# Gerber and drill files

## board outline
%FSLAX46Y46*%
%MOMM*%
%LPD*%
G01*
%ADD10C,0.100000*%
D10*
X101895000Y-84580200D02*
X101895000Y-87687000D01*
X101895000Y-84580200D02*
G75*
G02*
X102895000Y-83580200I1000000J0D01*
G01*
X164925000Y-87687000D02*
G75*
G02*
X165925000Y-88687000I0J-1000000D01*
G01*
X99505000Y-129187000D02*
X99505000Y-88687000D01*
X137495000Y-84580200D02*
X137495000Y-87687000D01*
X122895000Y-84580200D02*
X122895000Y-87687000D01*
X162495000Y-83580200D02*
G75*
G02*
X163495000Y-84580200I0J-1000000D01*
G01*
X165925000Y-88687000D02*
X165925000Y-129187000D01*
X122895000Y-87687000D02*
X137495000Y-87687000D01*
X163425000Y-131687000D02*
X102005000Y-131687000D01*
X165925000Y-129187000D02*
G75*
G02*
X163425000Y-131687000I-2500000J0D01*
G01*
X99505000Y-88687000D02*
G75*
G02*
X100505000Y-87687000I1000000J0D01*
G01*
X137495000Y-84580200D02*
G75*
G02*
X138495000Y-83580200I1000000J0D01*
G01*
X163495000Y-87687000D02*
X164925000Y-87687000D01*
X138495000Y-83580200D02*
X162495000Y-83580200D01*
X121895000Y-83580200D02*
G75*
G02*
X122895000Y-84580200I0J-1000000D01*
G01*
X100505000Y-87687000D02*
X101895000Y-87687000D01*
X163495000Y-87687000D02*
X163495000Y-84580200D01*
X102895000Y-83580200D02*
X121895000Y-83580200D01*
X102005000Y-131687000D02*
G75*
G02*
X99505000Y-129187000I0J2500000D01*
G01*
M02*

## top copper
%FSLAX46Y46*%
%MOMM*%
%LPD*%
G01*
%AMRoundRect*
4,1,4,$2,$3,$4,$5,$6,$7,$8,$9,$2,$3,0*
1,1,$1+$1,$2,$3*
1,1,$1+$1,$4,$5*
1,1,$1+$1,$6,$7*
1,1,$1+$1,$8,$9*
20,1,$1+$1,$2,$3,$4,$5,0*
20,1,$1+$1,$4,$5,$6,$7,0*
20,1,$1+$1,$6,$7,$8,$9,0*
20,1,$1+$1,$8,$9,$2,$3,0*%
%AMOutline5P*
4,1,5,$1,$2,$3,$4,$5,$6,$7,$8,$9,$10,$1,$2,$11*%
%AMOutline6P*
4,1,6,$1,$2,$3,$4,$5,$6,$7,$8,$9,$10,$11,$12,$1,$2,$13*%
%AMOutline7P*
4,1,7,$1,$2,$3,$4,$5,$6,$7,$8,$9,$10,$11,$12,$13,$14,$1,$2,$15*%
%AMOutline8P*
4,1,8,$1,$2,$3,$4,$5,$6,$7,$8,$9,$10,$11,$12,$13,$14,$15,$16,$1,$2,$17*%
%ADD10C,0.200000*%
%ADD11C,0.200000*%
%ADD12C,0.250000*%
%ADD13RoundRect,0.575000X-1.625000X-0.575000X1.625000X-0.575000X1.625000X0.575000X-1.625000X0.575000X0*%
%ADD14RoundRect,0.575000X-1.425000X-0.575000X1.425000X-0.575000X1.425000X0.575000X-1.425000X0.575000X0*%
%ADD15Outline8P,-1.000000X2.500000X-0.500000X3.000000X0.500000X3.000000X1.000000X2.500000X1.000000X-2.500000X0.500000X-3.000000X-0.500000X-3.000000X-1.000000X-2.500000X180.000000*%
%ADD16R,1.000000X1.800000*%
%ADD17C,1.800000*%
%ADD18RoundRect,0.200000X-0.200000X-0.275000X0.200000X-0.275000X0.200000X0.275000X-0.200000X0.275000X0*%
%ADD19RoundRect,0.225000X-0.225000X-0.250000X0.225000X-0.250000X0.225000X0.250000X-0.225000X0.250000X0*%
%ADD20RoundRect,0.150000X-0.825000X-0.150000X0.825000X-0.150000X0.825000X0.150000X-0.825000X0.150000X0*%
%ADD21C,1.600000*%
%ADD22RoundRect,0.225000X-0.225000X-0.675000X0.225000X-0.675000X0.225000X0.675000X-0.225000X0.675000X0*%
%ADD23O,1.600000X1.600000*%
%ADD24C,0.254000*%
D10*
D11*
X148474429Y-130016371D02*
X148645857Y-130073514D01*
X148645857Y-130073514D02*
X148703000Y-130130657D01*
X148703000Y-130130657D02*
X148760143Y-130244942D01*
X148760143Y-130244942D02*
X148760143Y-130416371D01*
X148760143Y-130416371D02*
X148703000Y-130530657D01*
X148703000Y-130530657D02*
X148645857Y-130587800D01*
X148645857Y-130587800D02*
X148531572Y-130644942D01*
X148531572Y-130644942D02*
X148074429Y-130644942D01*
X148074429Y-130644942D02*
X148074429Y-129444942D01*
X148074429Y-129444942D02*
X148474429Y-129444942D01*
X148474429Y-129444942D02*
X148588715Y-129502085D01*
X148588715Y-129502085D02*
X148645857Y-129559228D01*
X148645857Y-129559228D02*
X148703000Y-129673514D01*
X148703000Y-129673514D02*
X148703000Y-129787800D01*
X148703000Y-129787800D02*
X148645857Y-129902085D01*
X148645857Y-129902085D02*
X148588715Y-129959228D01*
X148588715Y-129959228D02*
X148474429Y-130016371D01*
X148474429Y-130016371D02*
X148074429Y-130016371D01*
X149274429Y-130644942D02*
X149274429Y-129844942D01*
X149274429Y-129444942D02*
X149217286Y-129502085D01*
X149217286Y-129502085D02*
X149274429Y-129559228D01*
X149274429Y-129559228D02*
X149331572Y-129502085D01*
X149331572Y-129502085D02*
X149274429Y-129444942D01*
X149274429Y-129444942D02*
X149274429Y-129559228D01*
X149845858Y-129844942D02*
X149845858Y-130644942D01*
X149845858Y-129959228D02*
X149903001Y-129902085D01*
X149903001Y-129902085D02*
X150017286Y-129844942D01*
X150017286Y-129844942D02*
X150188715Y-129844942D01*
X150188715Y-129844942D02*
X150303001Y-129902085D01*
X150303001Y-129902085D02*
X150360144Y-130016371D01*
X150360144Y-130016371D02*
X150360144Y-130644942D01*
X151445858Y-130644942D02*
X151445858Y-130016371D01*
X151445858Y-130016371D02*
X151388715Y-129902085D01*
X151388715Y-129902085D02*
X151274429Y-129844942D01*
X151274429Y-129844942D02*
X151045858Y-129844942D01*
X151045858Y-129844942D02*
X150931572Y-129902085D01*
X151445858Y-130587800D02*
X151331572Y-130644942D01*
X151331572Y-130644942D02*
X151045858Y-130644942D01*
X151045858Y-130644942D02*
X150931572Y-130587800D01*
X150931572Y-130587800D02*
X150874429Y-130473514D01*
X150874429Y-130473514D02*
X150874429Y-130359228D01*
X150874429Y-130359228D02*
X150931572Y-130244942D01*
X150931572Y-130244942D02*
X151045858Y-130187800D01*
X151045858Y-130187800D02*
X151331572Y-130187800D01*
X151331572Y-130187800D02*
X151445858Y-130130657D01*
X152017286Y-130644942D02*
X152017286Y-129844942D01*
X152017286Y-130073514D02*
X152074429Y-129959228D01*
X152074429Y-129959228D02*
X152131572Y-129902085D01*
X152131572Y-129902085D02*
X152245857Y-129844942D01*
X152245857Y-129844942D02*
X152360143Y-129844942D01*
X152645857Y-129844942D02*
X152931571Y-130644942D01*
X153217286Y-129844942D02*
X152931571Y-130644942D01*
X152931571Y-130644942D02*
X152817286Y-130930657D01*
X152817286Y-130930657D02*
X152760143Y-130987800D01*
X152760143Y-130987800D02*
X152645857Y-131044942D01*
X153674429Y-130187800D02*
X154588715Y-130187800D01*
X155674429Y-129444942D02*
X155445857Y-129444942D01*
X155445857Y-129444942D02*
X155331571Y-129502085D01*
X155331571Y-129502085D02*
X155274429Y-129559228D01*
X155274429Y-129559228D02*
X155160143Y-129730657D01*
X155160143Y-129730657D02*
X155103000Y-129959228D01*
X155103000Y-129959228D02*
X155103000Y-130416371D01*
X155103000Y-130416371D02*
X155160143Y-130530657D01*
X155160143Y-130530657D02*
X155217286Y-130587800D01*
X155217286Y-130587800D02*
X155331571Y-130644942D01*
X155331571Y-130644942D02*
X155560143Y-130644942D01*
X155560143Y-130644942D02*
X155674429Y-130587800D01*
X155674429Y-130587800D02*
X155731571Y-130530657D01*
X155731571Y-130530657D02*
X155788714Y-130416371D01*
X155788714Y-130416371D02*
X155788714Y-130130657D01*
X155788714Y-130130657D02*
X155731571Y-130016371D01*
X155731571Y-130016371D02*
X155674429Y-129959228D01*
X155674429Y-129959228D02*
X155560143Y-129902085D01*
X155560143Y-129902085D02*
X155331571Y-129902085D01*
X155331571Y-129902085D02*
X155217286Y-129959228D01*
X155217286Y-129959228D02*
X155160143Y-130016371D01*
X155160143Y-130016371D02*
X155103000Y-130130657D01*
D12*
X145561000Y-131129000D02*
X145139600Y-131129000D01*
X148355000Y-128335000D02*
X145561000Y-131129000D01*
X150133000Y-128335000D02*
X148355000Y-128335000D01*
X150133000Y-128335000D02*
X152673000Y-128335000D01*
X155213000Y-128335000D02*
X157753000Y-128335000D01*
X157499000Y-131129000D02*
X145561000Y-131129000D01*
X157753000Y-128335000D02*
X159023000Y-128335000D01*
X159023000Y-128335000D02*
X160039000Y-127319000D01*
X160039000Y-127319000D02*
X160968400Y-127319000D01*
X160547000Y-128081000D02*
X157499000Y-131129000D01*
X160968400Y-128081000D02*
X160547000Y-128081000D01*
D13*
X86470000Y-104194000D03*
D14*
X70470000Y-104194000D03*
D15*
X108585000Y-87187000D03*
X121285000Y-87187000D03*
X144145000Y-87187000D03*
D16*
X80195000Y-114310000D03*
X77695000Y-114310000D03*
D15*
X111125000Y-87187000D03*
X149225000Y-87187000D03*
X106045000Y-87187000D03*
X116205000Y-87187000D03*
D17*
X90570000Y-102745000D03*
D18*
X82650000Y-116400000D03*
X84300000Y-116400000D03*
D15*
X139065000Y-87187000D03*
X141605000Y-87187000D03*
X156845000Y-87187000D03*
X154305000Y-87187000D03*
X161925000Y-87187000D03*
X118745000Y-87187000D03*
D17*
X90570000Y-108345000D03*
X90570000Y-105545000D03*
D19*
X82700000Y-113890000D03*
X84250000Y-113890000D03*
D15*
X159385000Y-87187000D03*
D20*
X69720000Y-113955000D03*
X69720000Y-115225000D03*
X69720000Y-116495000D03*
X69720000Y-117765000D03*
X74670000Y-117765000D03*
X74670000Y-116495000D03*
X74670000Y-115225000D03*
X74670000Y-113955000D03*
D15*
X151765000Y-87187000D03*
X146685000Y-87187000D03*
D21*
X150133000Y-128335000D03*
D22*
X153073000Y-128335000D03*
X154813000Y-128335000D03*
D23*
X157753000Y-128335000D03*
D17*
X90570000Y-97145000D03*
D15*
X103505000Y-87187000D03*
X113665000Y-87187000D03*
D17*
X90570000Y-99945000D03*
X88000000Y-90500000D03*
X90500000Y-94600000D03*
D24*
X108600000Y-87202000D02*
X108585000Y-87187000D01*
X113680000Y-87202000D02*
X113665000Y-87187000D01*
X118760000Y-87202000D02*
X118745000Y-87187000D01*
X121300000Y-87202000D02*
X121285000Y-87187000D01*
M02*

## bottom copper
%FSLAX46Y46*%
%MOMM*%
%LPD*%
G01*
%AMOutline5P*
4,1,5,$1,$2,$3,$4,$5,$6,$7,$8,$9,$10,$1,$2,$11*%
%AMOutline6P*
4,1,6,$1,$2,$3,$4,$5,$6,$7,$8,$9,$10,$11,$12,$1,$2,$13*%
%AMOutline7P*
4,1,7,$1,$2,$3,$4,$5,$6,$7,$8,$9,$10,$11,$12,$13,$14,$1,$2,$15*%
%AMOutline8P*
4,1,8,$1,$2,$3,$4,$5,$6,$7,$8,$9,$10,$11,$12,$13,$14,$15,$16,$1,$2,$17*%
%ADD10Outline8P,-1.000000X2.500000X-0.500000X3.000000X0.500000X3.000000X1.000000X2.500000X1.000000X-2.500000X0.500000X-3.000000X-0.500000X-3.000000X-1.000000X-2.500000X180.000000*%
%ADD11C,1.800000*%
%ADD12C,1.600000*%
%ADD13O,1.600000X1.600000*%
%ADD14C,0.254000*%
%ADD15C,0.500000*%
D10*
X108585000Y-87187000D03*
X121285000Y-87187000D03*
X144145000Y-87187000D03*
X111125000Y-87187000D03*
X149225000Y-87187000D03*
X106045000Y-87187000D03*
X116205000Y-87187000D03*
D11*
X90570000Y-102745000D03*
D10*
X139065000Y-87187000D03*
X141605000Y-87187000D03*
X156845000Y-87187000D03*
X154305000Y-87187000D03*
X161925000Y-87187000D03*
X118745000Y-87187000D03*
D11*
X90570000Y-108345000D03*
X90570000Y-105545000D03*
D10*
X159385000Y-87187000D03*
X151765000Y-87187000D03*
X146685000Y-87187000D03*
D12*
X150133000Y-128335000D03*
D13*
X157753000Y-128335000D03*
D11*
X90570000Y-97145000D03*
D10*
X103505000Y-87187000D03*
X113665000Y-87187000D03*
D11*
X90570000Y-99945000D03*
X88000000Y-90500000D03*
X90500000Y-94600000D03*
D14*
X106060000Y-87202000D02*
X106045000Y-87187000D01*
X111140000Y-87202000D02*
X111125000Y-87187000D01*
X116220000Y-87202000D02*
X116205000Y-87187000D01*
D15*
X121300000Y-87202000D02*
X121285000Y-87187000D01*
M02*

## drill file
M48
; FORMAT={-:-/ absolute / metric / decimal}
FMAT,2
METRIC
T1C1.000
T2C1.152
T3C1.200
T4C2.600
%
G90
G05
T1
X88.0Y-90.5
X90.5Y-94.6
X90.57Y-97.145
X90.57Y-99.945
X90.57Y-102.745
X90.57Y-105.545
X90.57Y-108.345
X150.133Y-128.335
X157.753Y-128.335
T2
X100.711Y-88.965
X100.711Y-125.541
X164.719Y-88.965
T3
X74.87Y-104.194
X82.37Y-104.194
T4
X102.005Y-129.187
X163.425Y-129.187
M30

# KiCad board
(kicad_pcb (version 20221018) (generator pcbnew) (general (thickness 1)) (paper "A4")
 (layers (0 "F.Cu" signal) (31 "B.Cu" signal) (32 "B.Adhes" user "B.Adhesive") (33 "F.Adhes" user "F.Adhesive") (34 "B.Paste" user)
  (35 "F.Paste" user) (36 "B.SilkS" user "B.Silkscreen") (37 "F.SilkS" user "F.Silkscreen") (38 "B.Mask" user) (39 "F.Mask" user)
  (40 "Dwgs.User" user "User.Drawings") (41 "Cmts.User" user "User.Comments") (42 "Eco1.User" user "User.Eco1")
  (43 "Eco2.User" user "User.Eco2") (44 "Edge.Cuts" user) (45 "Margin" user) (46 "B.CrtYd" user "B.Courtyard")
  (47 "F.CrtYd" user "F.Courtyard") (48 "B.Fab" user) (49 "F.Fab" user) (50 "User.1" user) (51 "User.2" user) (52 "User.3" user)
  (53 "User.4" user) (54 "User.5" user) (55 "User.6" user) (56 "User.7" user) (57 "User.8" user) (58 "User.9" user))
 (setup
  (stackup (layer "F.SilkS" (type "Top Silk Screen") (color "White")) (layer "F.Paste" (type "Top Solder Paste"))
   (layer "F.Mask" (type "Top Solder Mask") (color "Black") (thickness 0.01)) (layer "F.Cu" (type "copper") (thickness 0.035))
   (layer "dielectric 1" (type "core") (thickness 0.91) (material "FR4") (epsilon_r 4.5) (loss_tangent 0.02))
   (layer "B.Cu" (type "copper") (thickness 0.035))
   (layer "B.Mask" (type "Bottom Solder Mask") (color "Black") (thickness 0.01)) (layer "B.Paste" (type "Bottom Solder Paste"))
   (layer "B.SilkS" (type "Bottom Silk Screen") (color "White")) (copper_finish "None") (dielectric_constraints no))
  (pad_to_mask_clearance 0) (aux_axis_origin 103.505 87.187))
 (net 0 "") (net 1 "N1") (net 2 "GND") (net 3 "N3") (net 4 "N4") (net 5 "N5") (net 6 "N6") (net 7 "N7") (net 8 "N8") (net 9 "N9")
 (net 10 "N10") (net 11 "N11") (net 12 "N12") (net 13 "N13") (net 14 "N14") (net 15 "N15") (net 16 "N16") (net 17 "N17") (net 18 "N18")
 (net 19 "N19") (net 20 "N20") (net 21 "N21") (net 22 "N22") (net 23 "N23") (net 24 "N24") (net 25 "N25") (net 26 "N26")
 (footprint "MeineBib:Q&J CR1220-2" (layer "F.Cu") (at 78.47 104.194)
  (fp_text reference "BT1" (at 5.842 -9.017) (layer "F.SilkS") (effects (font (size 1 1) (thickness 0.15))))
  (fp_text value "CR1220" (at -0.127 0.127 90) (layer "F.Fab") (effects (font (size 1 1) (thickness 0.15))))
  (pad "" np_thru_hole circle (at -3.6 0) (size 1.2 1.2) (drill 1.2) (layers "F&B.Cu" "*.Mask"))
  (pad "" np_thru_hole circle (at 3.9 0) (size 1.2 1.2) (drill 1.2) (layers "F&B.Cu" "*.Mask"))
  (pad "1" smd roundrect (at 8 0) (size 4.4 2.3) (layers "F.Cu" "F.Paste" "F.Mask") (roundrect_rratio 0.25) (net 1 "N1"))
  (pad "2" smd roundrect (at -8 0) (size 4 2.3) (layers "F.Cu" "F.Paste" "F.Mask") (roundrect_rratio 0.25) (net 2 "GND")))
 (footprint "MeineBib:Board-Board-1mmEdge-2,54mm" (layer "F.Cu") (at 108.585 87.187)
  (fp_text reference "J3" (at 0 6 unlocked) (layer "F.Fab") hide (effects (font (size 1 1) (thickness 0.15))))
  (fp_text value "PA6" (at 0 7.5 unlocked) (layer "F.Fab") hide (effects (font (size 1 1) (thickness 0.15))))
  (pad "1" smd roundrect (at 0 0 180) (size 2 6) (layers "F.Cu" "F.Paste" "F.Mask") (roundrect_rratio 0) (chamfer_ratio 0.25)
   (chamfer top_left top_right bottom_left bottom_right) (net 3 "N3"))
  (pad "1" smd roundrect (at 0 0 180) (size 2 6) (layers "B.Cu" "B.Paste" "B.Mask") (roundrect_rratio 0) (chamfer_ratio 0.25)
   (chamfer top_left top_right bottom_left bottom_right) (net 3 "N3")))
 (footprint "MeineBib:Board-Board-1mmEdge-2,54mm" (layer "F.Cu") (at 121.285 87.187)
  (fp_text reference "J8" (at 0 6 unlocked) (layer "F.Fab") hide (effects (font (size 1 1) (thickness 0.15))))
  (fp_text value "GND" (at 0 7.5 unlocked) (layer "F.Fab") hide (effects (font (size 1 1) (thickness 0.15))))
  (pad "1" smd roundrect (at 0 0 180) (size 2 6) (layers "F.Cu" "F.Paste" "F.Mask") (roundrect_rratio 0) (chamfer_ratio 0.25)
   (chamfer top_left top_right bottom_left bottom_right) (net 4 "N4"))
  (pad "1" smd roundrect (at 0 0 180) (size 2 6) (layers "B.Cu" "B.Paste" "B.Mask") (roundrect_rratio 0) (chamfer_ratio 0.25)
   (chamfer top_left top_right bottom_left bottom_right) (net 4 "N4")))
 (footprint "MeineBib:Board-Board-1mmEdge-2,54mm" (layer "F.Cu") (at 144.145 87.187)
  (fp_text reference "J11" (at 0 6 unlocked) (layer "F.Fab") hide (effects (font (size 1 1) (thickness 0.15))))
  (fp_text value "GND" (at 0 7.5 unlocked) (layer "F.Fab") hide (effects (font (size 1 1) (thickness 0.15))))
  (pad "1" smd roundrect (at 0 0 180) (size 2 6) (layers "F.Cu" "F.Paste" "F.Mask") (roundrect_rratio 0) (chamfer_ratio 0.25)
   (chamfer top_left top_right bottom_left bottom_right) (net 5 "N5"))
  (pad "1" smd roundrect (at 0 0 180) (size 2 6) (layers "B.Cu" "B.Paste" "B.Mask") (roundrect_rratio 0) (chamfer_ratio 0.25)
   (chamfer top_left top_right bottom_left bottom_right) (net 5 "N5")))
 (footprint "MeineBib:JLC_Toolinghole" (layer "F.Cu") (at 164.719 88.965)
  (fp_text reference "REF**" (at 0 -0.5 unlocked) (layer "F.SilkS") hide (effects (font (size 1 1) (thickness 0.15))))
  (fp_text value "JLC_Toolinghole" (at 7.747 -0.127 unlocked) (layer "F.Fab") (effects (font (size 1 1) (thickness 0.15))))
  (pad "" np_thru_hole circle (at 0 0) (size 1.3 1.3) (drill 1.152) (layers "*.Mask")))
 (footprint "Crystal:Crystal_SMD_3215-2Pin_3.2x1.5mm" (layer "F.Cu") (at 78.945 114.31)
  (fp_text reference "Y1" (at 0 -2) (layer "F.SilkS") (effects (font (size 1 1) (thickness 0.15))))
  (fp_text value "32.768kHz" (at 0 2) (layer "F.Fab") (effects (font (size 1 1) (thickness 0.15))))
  (pad "1" smd rect (at 1.25 0) (size 1 1.8) (layers "F.Cu" "F.Paste" "F.Mask") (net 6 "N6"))
  (pad "2" smd rect (at -1.25 0) (size 1 1.8) (layers "F.Cu" "F.Paste" "F.Mask") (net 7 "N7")))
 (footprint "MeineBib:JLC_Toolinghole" (layer "F.Cu") (at 100.711 125.541)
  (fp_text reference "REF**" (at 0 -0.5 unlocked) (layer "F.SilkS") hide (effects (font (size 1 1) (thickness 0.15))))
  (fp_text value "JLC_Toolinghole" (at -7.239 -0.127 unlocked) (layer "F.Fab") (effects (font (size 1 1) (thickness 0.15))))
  (pad "" np_thru_hole circle (at 0 0) (size 1.3 1.3) (drill 1.152) (layers "*.Mask")))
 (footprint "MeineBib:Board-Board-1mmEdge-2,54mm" (layer "F.Cu") (at 111.125 87.187)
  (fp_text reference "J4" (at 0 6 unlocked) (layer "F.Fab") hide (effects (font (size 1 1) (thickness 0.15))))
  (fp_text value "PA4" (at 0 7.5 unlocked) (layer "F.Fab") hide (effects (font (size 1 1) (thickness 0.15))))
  (pad "1" smd roundrect (at 0 0 180) (size 2 6) (layers "F.Cu" "F.Paste" "F.Mask") (roundrect_rratio 0) (chamfer_ratio 0.25)
   (chamfer top_left top_right bottom_left bottom_right) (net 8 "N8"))
  (pad "1" smd roundrect (at 0 0 180) (size 2 6) (layers "B.Cu" "B.Paste" "B.Mask") (roundrect_rratio 0) (chamfer_ratio 0.25)
   (chamfer top_left top_right bottom_left bottom_right) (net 8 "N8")))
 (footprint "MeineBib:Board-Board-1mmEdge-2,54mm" (layer "F.Cu") (at 149.225 87.187)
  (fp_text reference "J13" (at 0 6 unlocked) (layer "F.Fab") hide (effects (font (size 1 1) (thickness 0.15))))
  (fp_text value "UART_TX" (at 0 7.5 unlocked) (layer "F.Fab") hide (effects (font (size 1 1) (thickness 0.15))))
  (pad "1" smd roundrect (at 0 0 180) (size 2 6) (layers "F.Cu" "F.Paste" "F.Mask") (roundrect_rratio 0) (chamfer_ratio 0.25)
   (chamfer top_left top_right bottom_left bottom_right) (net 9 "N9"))
  (pad "1" smd roundrect (at 0 0 180) (size 2 6) (layers "B.Cu" "B.Paste" "B.Mask") (roundrect_rratio 0) (chamfer_ratio 0.25)
   (chamfer top_left top_right bottom_left bottom_right) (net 9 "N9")))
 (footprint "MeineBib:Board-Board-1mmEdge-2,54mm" (layer "F.Cu") (at 106.045 87.187)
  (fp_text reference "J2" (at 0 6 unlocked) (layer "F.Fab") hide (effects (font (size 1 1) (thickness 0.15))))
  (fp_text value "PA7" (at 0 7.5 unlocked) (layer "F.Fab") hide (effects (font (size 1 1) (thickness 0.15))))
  (pad "1" smd roundrect (at 0 0 180) (size 2 6) (layers "F.Cu" "F.Paste" "F.Mask") (roundrect_rratio 0) (chamfer_ratio 0.25)
   (chamfer top_left top_right bottom_left bottom_right) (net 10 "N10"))
  (pad "1" smd roundrect (at 0 0 180) (size 2 6) (layers "B.Cu" "B.Paste" "B.Mask") (roundrect_rratio 0) (chamfer_ratio 0.25)
   (chamfer top_left top_right bottom_left bottom_right) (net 10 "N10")))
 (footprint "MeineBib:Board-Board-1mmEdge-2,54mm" (layer "F.Cu") (at 116.205 87.187)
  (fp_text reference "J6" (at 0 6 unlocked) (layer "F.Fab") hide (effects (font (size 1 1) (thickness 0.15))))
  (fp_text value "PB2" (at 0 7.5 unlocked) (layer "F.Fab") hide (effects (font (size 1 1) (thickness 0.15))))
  (pad "1" smd roundrect (at 0 0 180) (size 2 6) (layers "F.Cu" "F.Paste" "F.Mask") (roundrect_rratio 0) (chamfer_ratio 0.25)
   (chamfer top_left top_right bottom_left bottom_right) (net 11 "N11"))
  (pad "1" smd roundrect (at 0 0 180) (size 2 6) (layers "B.Cu" "B.Paste" "B.Mask") (roundrect_rratio 0) (chamfer_ratio 0.25)
   (chamfer top_left top_right bottom_left bottom_right) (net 11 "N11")))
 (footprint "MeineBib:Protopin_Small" (layer "F.Cu") (at 90.57 102.745)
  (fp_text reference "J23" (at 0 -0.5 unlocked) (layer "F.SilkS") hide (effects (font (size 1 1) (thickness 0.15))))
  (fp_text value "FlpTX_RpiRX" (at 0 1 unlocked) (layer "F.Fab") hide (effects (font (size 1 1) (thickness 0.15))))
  (pad "1" thru_hole circle (at 0 0) (size 1.8 1.8) (drill 1) (layers "*.Cu" "*.Mask") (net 9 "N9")))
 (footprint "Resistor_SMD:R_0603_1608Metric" (layer "F.Cu") (at 83.475 116.4)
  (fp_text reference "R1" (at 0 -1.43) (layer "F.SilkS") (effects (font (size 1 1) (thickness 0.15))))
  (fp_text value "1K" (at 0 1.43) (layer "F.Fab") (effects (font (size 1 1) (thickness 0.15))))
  (pad "1" smd roundrect (at -0.825 0) (size 0.8 0.95) (layers "F.Cu" "F.Paste" "F.Mask") (roundrect_rratio 0.25) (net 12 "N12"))
  (pad "2" smd roundrect (at 0.825 0) (size 0.8 0.95) (layers "F.Cu" "F.Paste" "F.Mask") (roundrect_rratio 0.25) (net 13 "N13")))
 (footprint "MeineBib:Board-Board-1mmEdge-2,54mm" (layer "F.Cu") (at 139.065 87.187)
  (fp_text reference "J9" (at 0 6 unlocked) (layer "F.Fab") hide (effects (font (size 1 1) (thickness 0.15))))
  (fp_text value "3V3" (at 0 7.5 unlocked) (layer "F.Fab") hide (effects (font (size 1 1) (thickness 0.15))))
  (pad "1" smd roundrect (at 0 0 180) (size 2 6) (layers "F.Cu" "F.Paste" "F.Mask") (roundrect_rratio 0) (chamfer_ratio 0.25)
   (chamfer top_left top_right bottom_left bottom_right) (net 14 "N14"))
  (pad "1" smd roundrect (at 0 0 180) (size 2 6) (layers "B.Cu" "B.Paste" "B.Mask") (roundrect_rratio 0) (chamfer_ratio 0.25)
   (chamfer top_left top_right bottom_left bottom_right) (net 14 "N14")))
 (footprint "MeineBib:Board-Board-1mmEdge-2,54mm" (layer "F.Cu") (at 141.605 87.187)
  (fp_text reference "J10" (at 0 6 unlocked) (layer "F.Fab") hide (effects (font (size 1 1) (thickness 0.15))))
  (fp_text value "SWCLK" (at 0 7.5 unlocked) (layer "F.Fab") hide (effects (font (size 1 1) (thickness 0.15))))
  (pad "1" smd roundrect (at 0 0 180) (size 2 6) (layers "F.Cu" "F.Paste" "F.Mask") (roundrect_rratio 0) (chamfer_ratio 0.25)
   (chamfer top_left top_right bottom_left bottom_right) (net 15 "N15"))
  (pad "1" smd roundrect (at 0 0 180) (size 2 6) (layers "B.Cu" "B.Paste" "B.Mask") (roundrect_rratio 0) (chamfer_ratio 0.25)
   (chamfer top_left top_right bottom_left bottom_right) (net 15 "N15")))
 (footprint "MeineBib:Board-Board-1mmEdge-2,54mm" (layer "F.Cu") (at 156.845 87.187)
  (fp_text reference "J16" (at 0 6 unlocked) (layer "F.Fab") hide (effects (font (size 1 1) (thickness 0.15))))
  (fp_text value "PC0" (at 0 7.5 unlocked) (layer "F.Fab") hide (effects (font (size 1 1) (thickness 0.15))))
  (pad "1" smd roundrect (at 0 0 180) (size 2 6) (layers "F.Cu" "F.Paste" "F.Mask") (roundrect_rratio 0) (chamfer_ratio 0.25)
   (chamfer top_left top_right bottom_left bottom_right) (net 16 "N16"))
  (pad "1" smd roundrect (at 0 0 180) (size 2 6) (layers "B.Cu" "B.Paste" "B.Mask") (roundrect_rratio 0) (chamfer_ratio 0.25)
   (chamfer top_left top_right bottom_left bottom_right) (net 16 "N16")))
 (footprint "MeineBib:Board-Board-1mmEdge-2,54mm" (layer "F.Cu") (at 154.305 87.187)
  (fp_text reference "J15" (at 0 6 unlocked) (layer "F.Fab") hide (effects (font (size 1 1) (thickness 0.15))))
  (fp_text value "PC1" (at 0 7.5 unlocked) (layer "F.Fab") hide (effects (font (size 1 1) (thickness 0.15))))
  (pad "1" smd roundrect (at 0 0 180) (size 2 6) (layers "F.Cu" "F.Paste" "F.Mask") (roundrect_rratio 0) (chamfer_ratio 0.25)
   (chamfer top_left top_right bottom_left bottom_right) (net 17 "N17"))
  (pad "1" smd roundrect (at 0 0 180) (size 2 6) (layers "B.Cu" "B.Paste" "B.Mask") (roundrect_rratio 0) (chamfer_ratio 0.25)
   (chamfer top_left top_right bottom_left bottom_right) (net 17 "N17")))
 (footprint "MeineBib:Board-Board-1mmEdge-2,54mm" (layer "F.Cu") (at 161.925 87.187)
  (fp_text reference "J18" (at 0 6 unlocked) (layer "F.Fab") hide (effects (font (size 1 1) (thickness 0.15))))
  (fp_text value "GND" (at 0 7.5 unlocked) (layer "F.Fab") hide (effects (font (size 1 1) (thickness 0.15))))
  (pad "1" smd roundrect (at 0 0 180) (size 2 6) (layers "F.Cu" "F.Paste" "F.Mask") (roundrect_rratio 0) (chamfer_ratio 0.25)
   (chamfer top_left top_right bottom_left bottom_right) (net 2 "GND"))
  (pad "1" smd roundrect (at 0 0 180) (size 2 6) (layers "B.Cu" "B.Paste" "B.Mask") (roundrect_rratio 0) (chamfer_ratio 0.25)
   (chamfer top_left top_right bottom_left bottom_right) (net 2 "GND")))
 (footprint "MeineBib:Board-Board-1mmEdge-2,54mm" (layer "F.Cu") (at 118.745 87.187)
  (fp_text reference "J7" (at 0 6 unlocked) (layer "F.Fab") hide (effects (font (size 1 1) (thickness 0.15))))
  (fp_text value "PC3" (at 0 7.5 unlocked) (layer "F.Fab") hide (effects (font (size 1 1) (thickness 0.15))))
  (pad "1" smd roundrect (at 0 0 180) (size 2 6) (layers "F.Cu" "F.Paste" "F.Mask") (roundrect_rratio 0) (chamfer_ratio 0.25)
   (chamfer top_left top_right bottom_left bottom_right) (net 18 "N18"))
  (pad "1" smd roundrect (at 0 0 180) (size 2 6) (layers "B.Cu" "B.Paste" "B.Mask") (roundrect_rratio 0) (chamfer_ratio 0.25)
   (chamfer top_left top_right bottom_left bottom_right) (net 18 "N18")))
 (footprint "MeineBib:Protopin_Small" (layer "F.Cu") (at 90.57 108.345)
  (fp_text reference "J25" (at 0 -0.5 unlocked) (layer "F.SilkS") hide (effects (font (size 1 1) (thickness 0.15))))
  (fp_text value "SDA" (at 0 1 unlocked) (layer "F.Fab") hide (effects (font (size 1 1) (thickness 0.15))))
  (pad "1" thru_hole circle (at 0 0) (size 1.8 1.8) (drill 1) (layers "*.Cu" "*.Mask") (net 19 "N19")))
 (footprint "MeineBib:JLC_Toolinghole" (layer "F.Cu") (at 100.711 88.965)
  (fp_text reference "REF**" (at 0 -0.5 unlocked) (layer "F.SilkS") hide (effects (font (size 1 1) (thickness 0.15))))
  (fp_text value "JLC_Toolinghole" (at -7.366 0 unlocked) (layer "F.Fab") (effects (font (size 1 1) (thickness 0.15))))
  (pad "" np_thru_hole circle (at 0 0) (size 1.3 1.3) (drill 1.152) (layers "*.Mask")))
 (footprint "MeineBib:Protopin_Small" (layer "F.Cu") (at 90.57 105.545)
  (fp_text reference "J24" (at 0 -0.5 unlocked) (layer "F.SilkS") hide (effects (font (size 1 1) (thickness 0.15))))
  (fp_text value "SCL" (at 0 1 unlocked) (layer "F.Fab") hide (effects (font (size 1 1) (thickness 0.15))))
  (pad "1" thru_hole circle (at 0 0) (size 1.8 1.8) (drill 1) (layers "*.Cu" "*.Mask") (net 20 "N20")))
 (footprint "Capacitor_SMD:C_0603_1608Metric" (layer "F.Cu") (at 83.475 113.89)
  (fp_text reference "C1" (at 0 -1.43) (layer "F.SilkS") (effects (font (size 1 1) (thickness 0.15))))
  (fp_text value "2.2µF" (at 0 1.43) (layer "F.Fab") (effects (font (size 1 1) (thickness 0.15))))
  (pad "1" smd roundrect (at -0.775 0) (size 0.9 0.95) (layers "F.Cu" "F.Paste" "F.Mask") (roundrect_rratio 0.25) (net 13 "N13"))
  (pad "2" smd roundrect (at 0.775 0) (size 0.9 0.95) (layers "F.Cu" "F.Paste" "F.Mask") (roundrect_rratio 0.25) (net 2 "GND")))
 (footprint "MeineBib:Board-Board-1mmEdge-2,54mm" (layer "F.Cu") (at 159.385 87.187)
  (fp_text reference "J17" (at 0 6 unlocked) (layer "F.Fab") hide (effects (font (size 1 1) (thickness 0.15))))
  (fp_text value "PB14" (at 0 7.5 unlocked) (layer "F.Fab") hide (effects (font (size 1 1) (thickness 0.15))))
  (pad "1" smd roundrect (at 0 0 180) (size 2 6) (layers "F.Cu" "F.Paste" "F.Mask") (roundrect_rratio 0) (chamfer_ratio 0.25)
   (chamfer top_left top_right bottom_left bottom_right) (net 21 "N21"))
  (pad "1" smd roundrect (at 0 0 180) (size 2 6) (layers "B.Cu" "B.Paste" "B.Mask") (roundrect_rratio 0) (chamfer_ratio 0.25)
   (chamfer top_left top_right bottom_left bottom_right) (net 21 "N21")))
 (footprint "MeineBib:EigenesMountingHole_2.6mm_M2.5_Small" (layer "F.Cu") (at 102.005 129.187)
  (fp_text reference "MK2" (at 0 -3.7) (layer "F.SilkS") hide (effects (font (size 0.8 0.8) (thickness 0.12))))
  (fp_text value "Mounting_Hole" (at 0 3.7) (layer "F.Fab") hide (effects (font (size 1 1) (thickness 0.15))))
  (pad "" np_thru_hole circle (at 0 0) (size 2.6 2.6) (drill 2.6) (layers "F&B.Cu" "*.Mask") (solder_mask_margin 1.25) (clearance 1.25)))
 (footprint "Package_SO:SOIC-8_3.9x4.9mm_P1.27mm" (layer "F.Cu") (at 72.195 115.86)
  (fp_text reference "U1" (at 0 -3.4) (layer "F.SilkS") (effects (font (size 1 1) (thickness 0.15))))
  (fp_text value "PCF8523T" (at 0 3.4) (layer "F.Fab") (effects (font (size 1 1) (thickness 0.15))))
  (pad "1" smd roundrect (at -2.475 -1.905) (size 1.95 0.6) (layers "F.Cu" "F.Paste" "F.Mask") (roundrect_rratio 0.25) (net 6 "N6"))
  (pad "2" smd roundrect (at -2.475 -0.635) (size 1.95 0.6) (layers "F.Cu" "F.Paste" "F.Mask") (roundrect_rratio 0.25) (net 7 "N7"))
  (pad "3" smd roundrect (at -2.475 0.635) (size 1.95 0.6) (layers "F.Cu" "F.Paste" "F.Mask") (roundrect_rratio 0.25) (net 1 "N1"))
  (pad "4" smd roundrect (at -2.475 1.905) (size 1.95 0.6) (layers "F.Cu" "F.Paste" "F.Mask") (roundrect_rratio 0.25) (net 2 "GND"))
  (pad "5" smd roundrect (at 2.475 1.905) (size 1.95 0.6) (layers "F.Cu" "F.Paste" "F.Mask") (roundrect_rratio 0.25) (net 19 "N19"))
  (pad "6" smd roundrect (at 2.475 0.635) (size 1.95 0.6) (layers "F.Cu" "F.Paste" "F.Mask") (roundrect_rratio 0.25) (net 20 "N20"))
  (pad "7" smd roundrect (at 2.475 -0.635) (size 1.95 0.6) (layers "F.Cu" "F.Paste" "F.Mask") (roundrect_rratio 0.25) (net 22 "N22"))
  (pad "8" smd roundrect (at 2.475 -1.905) (size 1.95 0.6) (layers "F.Cu" "F.Paste" "F.Mask") (roundrect_rratio 0.25) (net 13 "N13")))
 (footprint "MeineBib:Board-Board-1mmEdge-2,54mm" (layer "F.Cu") (at 151.765 87.187)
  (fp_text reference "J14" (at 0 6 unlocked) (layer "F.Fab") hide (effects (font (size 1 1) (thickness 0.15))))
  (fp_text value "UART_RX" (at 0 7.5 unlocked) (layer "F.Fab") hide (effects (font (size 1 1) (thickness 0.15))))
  (pad "1" smd roundrect (at 0 0 180) (size 2 6) (layers "F.Cu" "F.Paste" "F.Mask") (roundrect_rratio 0) (chamfer_ratio 0.25)
   (chamfer top_left top_right bottom_left bottom_right) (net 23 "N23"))
  (pad "1" smd roundrect (at 0 0 180) (size 2 6) (layers "B.Cu" "B.Paste" "B.Mask") (roundrect_rratio 0) (chamfer_ratio 0.25)
   (chamfer top_left top_right bottom_left bottom_right) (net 23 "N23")))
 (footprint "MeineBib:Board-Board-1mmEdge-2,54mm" (layer "F.Cu") (at 146.685 87.187)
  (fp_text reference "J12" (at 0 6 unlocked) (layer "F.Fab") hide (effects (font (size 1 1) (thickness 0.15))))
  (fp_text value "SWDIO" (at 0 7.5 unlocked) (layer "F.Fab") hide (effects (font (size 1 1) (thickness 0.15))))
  (pad "1" smd roundrect (at 0 0 180) (size 2 6) (layers "F.Cu" "F.Paste" "F.Mask") (roundrect_rratio 0) (chamfer_ratio 0.25)
   (chamfer top_left top_right bottom_left bottom_right) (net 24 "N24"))
  (pad "1" smd roundrect (at 0 0 180) (size 2 6) (layers "B.Cu" "B.Paste" "B.Mask") (roundrect_rratio 0) (chamfer_ratio 0.25)
   (chamfer top_left top_right bottom_left bottom_right) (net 24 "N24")))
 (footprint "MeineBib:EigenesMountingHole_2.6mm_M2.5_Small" (layer "F.Cu") (at 163.425 129.187)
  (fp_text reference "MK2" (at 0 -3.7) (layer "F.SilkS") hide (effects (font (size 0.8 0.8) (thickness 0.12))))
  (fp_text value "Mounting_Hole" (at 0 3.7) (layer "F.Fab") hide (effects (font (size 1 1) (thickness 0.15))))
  (pad "" np_thru_hole circle (at 0 0) (size 2.6 2.6) (drill 2.6) (layers "F&B.Cu" "*.Mask") (solder_mask_margin 1.25) (clearance 1.25)))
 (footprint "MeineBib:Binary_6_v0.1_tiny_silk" (layer "F.Cu") (at 153.9684 129.3002) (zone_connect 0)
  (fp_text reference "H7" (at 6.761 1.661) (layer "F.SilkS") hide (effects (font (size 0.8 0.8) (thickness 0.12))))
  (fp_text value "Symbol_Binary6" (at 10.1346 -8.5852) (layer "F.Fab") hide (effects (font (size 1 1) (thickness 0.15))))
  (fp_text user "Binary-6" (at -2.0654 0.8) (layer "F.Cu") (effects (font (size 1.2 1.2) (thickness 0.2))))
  (fp_line (start -8.4074 1.8288) (end -8.8288 1.8288) (stroke (width 0.25) (type solid)) (layer "F.Cu"))
  (fp_line (start -5.6134 -0.9652) (end -8.4074 1.8288) (stroke (width 0.25) (type solid)) (layer "F.Cu"))
  (fp_line (start -3.8354 -0.9652) (end -5.6134 -0.9652) (stroke (width 0.25) (type solid)) (layer "F.Cu"))
  (fp_line (start -3.8354 -0.9652) (end -1.2954 -0.9652) (stroke (width 0.25) (type solid)) (layer "F.Cu"))
  (fp_line (start 1.2446 -0.9652) (end 3.7846 -0.9652) (stroke (width 0.25) (type solid)) (layer "F.Cu"))
  (fp_line (start 3.5306 1.8288) (end -8.4074 1.8288) (stroke (width 0.25) (type solid)) (layer "F.Cu"))
  (fp_line (start 3.7846 -0.9652) (end 5.0546 -0.9652) (stroke (width 0.25) (type solid)) (layer "F.Cu"))
  (fp_line (start 5.0546 -0.9652) (end 6.0706 -1.9812) (stroke (width 0.25) (type solid)) (layer "F.Cu"))
  (fp_line (start 6.0706 -1.9812) (end 7 -1.9812) (stroke (width 0.25) (type solid)) (layer "F.Cu"))
  (fp_line (start 6.5786 -1.2192) (end 3.5306 1.8288) (stroke (width 0.25) (type solid)) (layer "F.Cu"))
  (fp_line (start 7 -1.2192) (end 6.5786 -1.2192) (stroke (width 0.25) (type solid)) (layer "F.Cu"))
  (pad "" thru_hole circle (at -3.8354 -0.9652) (size 1.6 1.6) (drill 1) (layers "*.Cu" "*.Mask") (zone_connect 0))
  (pad "" smd roundrect (at -0.8954 -0.9652) (size 0.9 1.8) (layers "F.Cu" "F.Mask") (roundrect_rratio 0.25) (zone_connect 0))
  (pad "" smd roundrect (at 0.8446 -0.9652) (size 0.9 1.8) (layers "F.Cu" "F.Mask") (roundrect_rratio 0.25) (zone_connect 0))
  (pad "" thru_hole oval (at 3.7846 -0.9652) (size 1.6 1.6) (drill 1) (layers "*.Cu" "*.Mask") (zone_connect 0)))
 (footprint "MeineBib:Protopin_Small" (layer "F.Cu") (at 90.57 97.145)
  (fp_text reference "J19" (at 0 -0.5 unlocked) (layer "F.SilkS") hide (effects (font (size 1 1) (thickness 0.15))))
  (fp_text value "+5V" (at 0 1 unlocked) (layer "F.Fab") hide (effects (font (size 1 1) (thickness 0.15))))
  (pad "1" thru_hole circle (at 0 0) (size 1.8 1.8) (drill 1) (layers "*.Cu" "*.Mask") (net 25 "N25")))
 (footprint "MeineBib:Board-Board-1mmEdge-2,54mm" (layer "F.Cu") (at 103.505 87.187)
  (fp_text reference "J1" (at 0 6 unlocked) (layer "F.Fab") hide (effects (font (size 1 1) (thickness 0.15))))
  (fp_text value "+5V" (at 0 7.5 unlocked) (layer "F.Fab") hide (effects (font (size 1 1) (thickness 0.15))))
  (pad "1" smd roundrect (at 0 0 180) (size 2 6) (layers "F.Cu" "F.Paste" "F.Mask") (roundrect_rratio 0) (chamfer_ratio 0.25)
   (chamfer top_left top_right bottom_left bottom_right) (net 25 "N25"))
  (pad "1" smd roundrect (at 0 0 180) (size 2 6) (layers "B.Cu" "B.Paste" "B.Mask") (roundrect_rratio 0) (chamfer_ratio 0.25)
   (chamfer top_left top_right bottom_left bottom_right) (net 25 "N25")))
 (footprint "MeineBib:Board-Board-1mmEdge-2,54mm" (layer "F.Cu") (at 113.665 87.187)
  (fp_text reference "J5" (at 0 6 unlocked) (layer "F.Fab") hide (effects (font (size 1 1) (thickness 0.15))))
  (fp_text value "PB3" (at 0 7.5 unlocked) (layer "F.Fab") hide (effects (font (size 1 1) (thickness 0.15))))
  (pad "1" smd roundrect (at 0 0 180) (size 2 6) (layers "F.Cu" "F.Paste" "F.Mask") (roundrect_rratio 0) (chamfer_ratio 0.25)
   (chamfer top_left top_right bottom_left bottom_right) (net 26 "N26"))
  (pad "1" smd roundrect (at 0 0 180) (size 2 6) (layers "B.Cu" "B.Paste" "B.Mask") (roundrect_rratio 0) (chamfer_ratio 0.25)
   (chamfer top_left top_right bottom_left bottom_right) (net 26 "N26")))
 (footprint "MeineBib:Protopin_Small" (layer "F.Cu") (at 90.57 99.945)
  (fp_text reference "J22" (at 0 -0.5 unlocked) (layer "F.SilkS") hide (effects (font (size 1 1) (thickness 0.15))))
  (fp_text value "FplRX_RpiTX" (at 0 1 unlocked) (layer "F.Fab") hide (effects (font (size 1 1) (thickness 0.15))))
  (pad "1" thru_hole circle (at 0 0) (size 1.8 1.8) (drill 1) (layers "*.Cu" "*.Mask") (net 23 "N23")))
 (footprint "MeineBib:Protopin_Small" (layer "B.Cu") (at 88 90.5 -90)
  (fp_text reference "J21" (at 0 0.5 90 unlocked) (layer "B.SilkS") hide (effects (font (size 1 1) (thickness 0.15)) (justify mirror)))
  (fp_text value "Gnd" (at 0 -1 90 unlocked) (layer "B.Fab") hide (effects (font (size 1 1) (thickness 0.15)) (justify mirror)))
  (pad "1" thru_hole circle (at 0 0 270) (size 1.8 1.8) (drill 1) (layers "*.Cu" "*.Mask") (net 2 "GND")))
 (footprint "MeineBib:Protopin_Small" (layer "B.Cu") (at 90.5 94.6 -90)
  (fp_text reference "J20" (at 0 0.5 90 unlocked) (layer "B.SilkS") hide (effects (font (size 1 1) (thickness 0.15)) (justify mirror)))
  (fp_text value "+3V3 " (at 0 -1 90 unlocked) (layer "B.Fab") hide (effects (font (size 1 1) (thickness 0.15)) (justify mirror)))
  (pad "1" thru_hole circle (at 0 0 270) (size 1.8 1.8) (drill 1) (layers "*.Cu" "*.Mask") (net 12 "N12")))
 (gr_line (start 101.895 84.5802) (end 101.895 87.687) (stroke (width 0.1) (type solid)) (layer "Edge.Cuts"))
 (gr_arc (start 101.895 84.5802) (mid 102.187893 83.873093) (end 102.895 83.5802) (stroke (width 0.1) (type solid)) (layer "Edge.Cuts"))
 (gr_arc (start 164.925 87.687) (mid 165.632107 87.979893) (end 165.925 88.687) (stroke (width 0.1) (type solid)) (layer "Edge.Cuts"))
 (gr_line (start 99.505 129.187) (end 99.505 88.687) (stroke (width 0.1) (type solid)) (layer "Edge.Cuts"))
 (gr_line (start 137.495 84.5802) (end 137.495 87.687) (stroke (width 0.1) (type solid)) (layer "Edge.Cuts"))
 (gr_line (start 122.895 84.5802) (end 122.895 87.687) (stroke (width 0.1) (type solid)) (layer "Edge.Cuts"))
 (gr_arc (start 162.495 83.5802) (mid 163.202107 83.873093) (end 163.495 84.5802) (stroke (width 0.1) (type solid)) (layer "Edge.Cuts"))
 (gr_line (start 165.925 88.687) (end 165.925 129.187) (stroke (width 0.1) (type solid)) (layer "Edge.Cuts"))
 (gr_line (start 122.895 87.687) (end 137.495 87.687) (stroke (width 0.1) (type solid)) (layer "Edge.Cuts"))
 (gr_line (start 163.425 131.687) (end 102.005 131.687) (stroke (width 0.1) (type solid)) (layer "Edge.Cuts"))
 (gr_arc (start 165.925 129.187) (mid 165.192767 130.954767) (end 163.425 131.687) (stroke (width 0.1) (type solid)) (layer "Edge.Cuts"))
 (gr_arc (start 99.505 88.687) (mid 99.797893 87.979893) (end 100.505 87.687) (stroke (width 0.1) (type solid)) (layer "Edge.Cuts"))
 (gr_arc (start 137.495 84.5802) (mid 137.787893 83.873093) (end 138.495 83.5802) (stroke (width 0.1) (type solid)) (layer "Edge.Cuts"))
 (gr_line (start 163.495 87.687) (end 164.925 87.687) (stroke (width 0.1) (type solid)) (layer "Edge.Cuts"))
 (gr_line (start 138.495 83.5802) (end 162.495 83.5802) (stroke (width 0.1) (type solid)) (layer "Edge.Cuts"))
 (gr_arc (start 121.895 83.5802) (mid 122.602107 83.873093) (end 122.895 84.5802) (stroke (width 0.1) (type solid)) (layer "Edge.Cuts"))
 (gr_line (start 100.505 87.687) (end 101.895 87.687) (stroke (width 0.1) (type solid)) (layer "Edge.Cuts"))
 (gr_line (start 163.495 87.687) (end 163.495 84.5802) (stroke (width 0.1) (type solid)) (layer "Edge.Cuts"))
 (gr_line (start 102.895 83.5802) (end 121.895 83.5802) (stroke (width 0.1) (type solid)) (layer "Edge.Cuts"))
 (gr_arc (start 102.005 131.687) (mid 100.237233 130.954767) (end 99.505 129.187) (stroke (width 0.1) (type solid)) (layer "Edge.Cuts"))
 (segment (start 106.06 87.202) (end 106.045 87.187) (width 0.254) (layer "B.Cu") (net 10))
 (segment (start 108.6 87.202) (end 108.585 87.187) (width 0.254) (layer "F.Cu") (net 3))
 (segment (start 111.14 87.202) (end 111.125 87.187) (width 0.254) (layer "B.Cu") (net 8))
 (segment (start 113.68 87.202) (end 113.665 87.187) (width 0.254) (layer "F.Cu") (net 26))
 (segment (start 116.22 87.202) (end 116.205 87.187) (width 0.254) (layer "B.Cu") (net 11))
 (segment (start 118.76 87.202) (end 118.745 87.187) (width 0.254) (layer "F.Cu") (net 18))
 (segment (start 121.3 87.202) (end 121.285 87.187) (width 0.254) (layer "F.Cu") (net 4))
 (segment (start 121.3 87.202) (end 121.285 87.187) (width 0.5) (layer "B.Cu") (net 4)))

